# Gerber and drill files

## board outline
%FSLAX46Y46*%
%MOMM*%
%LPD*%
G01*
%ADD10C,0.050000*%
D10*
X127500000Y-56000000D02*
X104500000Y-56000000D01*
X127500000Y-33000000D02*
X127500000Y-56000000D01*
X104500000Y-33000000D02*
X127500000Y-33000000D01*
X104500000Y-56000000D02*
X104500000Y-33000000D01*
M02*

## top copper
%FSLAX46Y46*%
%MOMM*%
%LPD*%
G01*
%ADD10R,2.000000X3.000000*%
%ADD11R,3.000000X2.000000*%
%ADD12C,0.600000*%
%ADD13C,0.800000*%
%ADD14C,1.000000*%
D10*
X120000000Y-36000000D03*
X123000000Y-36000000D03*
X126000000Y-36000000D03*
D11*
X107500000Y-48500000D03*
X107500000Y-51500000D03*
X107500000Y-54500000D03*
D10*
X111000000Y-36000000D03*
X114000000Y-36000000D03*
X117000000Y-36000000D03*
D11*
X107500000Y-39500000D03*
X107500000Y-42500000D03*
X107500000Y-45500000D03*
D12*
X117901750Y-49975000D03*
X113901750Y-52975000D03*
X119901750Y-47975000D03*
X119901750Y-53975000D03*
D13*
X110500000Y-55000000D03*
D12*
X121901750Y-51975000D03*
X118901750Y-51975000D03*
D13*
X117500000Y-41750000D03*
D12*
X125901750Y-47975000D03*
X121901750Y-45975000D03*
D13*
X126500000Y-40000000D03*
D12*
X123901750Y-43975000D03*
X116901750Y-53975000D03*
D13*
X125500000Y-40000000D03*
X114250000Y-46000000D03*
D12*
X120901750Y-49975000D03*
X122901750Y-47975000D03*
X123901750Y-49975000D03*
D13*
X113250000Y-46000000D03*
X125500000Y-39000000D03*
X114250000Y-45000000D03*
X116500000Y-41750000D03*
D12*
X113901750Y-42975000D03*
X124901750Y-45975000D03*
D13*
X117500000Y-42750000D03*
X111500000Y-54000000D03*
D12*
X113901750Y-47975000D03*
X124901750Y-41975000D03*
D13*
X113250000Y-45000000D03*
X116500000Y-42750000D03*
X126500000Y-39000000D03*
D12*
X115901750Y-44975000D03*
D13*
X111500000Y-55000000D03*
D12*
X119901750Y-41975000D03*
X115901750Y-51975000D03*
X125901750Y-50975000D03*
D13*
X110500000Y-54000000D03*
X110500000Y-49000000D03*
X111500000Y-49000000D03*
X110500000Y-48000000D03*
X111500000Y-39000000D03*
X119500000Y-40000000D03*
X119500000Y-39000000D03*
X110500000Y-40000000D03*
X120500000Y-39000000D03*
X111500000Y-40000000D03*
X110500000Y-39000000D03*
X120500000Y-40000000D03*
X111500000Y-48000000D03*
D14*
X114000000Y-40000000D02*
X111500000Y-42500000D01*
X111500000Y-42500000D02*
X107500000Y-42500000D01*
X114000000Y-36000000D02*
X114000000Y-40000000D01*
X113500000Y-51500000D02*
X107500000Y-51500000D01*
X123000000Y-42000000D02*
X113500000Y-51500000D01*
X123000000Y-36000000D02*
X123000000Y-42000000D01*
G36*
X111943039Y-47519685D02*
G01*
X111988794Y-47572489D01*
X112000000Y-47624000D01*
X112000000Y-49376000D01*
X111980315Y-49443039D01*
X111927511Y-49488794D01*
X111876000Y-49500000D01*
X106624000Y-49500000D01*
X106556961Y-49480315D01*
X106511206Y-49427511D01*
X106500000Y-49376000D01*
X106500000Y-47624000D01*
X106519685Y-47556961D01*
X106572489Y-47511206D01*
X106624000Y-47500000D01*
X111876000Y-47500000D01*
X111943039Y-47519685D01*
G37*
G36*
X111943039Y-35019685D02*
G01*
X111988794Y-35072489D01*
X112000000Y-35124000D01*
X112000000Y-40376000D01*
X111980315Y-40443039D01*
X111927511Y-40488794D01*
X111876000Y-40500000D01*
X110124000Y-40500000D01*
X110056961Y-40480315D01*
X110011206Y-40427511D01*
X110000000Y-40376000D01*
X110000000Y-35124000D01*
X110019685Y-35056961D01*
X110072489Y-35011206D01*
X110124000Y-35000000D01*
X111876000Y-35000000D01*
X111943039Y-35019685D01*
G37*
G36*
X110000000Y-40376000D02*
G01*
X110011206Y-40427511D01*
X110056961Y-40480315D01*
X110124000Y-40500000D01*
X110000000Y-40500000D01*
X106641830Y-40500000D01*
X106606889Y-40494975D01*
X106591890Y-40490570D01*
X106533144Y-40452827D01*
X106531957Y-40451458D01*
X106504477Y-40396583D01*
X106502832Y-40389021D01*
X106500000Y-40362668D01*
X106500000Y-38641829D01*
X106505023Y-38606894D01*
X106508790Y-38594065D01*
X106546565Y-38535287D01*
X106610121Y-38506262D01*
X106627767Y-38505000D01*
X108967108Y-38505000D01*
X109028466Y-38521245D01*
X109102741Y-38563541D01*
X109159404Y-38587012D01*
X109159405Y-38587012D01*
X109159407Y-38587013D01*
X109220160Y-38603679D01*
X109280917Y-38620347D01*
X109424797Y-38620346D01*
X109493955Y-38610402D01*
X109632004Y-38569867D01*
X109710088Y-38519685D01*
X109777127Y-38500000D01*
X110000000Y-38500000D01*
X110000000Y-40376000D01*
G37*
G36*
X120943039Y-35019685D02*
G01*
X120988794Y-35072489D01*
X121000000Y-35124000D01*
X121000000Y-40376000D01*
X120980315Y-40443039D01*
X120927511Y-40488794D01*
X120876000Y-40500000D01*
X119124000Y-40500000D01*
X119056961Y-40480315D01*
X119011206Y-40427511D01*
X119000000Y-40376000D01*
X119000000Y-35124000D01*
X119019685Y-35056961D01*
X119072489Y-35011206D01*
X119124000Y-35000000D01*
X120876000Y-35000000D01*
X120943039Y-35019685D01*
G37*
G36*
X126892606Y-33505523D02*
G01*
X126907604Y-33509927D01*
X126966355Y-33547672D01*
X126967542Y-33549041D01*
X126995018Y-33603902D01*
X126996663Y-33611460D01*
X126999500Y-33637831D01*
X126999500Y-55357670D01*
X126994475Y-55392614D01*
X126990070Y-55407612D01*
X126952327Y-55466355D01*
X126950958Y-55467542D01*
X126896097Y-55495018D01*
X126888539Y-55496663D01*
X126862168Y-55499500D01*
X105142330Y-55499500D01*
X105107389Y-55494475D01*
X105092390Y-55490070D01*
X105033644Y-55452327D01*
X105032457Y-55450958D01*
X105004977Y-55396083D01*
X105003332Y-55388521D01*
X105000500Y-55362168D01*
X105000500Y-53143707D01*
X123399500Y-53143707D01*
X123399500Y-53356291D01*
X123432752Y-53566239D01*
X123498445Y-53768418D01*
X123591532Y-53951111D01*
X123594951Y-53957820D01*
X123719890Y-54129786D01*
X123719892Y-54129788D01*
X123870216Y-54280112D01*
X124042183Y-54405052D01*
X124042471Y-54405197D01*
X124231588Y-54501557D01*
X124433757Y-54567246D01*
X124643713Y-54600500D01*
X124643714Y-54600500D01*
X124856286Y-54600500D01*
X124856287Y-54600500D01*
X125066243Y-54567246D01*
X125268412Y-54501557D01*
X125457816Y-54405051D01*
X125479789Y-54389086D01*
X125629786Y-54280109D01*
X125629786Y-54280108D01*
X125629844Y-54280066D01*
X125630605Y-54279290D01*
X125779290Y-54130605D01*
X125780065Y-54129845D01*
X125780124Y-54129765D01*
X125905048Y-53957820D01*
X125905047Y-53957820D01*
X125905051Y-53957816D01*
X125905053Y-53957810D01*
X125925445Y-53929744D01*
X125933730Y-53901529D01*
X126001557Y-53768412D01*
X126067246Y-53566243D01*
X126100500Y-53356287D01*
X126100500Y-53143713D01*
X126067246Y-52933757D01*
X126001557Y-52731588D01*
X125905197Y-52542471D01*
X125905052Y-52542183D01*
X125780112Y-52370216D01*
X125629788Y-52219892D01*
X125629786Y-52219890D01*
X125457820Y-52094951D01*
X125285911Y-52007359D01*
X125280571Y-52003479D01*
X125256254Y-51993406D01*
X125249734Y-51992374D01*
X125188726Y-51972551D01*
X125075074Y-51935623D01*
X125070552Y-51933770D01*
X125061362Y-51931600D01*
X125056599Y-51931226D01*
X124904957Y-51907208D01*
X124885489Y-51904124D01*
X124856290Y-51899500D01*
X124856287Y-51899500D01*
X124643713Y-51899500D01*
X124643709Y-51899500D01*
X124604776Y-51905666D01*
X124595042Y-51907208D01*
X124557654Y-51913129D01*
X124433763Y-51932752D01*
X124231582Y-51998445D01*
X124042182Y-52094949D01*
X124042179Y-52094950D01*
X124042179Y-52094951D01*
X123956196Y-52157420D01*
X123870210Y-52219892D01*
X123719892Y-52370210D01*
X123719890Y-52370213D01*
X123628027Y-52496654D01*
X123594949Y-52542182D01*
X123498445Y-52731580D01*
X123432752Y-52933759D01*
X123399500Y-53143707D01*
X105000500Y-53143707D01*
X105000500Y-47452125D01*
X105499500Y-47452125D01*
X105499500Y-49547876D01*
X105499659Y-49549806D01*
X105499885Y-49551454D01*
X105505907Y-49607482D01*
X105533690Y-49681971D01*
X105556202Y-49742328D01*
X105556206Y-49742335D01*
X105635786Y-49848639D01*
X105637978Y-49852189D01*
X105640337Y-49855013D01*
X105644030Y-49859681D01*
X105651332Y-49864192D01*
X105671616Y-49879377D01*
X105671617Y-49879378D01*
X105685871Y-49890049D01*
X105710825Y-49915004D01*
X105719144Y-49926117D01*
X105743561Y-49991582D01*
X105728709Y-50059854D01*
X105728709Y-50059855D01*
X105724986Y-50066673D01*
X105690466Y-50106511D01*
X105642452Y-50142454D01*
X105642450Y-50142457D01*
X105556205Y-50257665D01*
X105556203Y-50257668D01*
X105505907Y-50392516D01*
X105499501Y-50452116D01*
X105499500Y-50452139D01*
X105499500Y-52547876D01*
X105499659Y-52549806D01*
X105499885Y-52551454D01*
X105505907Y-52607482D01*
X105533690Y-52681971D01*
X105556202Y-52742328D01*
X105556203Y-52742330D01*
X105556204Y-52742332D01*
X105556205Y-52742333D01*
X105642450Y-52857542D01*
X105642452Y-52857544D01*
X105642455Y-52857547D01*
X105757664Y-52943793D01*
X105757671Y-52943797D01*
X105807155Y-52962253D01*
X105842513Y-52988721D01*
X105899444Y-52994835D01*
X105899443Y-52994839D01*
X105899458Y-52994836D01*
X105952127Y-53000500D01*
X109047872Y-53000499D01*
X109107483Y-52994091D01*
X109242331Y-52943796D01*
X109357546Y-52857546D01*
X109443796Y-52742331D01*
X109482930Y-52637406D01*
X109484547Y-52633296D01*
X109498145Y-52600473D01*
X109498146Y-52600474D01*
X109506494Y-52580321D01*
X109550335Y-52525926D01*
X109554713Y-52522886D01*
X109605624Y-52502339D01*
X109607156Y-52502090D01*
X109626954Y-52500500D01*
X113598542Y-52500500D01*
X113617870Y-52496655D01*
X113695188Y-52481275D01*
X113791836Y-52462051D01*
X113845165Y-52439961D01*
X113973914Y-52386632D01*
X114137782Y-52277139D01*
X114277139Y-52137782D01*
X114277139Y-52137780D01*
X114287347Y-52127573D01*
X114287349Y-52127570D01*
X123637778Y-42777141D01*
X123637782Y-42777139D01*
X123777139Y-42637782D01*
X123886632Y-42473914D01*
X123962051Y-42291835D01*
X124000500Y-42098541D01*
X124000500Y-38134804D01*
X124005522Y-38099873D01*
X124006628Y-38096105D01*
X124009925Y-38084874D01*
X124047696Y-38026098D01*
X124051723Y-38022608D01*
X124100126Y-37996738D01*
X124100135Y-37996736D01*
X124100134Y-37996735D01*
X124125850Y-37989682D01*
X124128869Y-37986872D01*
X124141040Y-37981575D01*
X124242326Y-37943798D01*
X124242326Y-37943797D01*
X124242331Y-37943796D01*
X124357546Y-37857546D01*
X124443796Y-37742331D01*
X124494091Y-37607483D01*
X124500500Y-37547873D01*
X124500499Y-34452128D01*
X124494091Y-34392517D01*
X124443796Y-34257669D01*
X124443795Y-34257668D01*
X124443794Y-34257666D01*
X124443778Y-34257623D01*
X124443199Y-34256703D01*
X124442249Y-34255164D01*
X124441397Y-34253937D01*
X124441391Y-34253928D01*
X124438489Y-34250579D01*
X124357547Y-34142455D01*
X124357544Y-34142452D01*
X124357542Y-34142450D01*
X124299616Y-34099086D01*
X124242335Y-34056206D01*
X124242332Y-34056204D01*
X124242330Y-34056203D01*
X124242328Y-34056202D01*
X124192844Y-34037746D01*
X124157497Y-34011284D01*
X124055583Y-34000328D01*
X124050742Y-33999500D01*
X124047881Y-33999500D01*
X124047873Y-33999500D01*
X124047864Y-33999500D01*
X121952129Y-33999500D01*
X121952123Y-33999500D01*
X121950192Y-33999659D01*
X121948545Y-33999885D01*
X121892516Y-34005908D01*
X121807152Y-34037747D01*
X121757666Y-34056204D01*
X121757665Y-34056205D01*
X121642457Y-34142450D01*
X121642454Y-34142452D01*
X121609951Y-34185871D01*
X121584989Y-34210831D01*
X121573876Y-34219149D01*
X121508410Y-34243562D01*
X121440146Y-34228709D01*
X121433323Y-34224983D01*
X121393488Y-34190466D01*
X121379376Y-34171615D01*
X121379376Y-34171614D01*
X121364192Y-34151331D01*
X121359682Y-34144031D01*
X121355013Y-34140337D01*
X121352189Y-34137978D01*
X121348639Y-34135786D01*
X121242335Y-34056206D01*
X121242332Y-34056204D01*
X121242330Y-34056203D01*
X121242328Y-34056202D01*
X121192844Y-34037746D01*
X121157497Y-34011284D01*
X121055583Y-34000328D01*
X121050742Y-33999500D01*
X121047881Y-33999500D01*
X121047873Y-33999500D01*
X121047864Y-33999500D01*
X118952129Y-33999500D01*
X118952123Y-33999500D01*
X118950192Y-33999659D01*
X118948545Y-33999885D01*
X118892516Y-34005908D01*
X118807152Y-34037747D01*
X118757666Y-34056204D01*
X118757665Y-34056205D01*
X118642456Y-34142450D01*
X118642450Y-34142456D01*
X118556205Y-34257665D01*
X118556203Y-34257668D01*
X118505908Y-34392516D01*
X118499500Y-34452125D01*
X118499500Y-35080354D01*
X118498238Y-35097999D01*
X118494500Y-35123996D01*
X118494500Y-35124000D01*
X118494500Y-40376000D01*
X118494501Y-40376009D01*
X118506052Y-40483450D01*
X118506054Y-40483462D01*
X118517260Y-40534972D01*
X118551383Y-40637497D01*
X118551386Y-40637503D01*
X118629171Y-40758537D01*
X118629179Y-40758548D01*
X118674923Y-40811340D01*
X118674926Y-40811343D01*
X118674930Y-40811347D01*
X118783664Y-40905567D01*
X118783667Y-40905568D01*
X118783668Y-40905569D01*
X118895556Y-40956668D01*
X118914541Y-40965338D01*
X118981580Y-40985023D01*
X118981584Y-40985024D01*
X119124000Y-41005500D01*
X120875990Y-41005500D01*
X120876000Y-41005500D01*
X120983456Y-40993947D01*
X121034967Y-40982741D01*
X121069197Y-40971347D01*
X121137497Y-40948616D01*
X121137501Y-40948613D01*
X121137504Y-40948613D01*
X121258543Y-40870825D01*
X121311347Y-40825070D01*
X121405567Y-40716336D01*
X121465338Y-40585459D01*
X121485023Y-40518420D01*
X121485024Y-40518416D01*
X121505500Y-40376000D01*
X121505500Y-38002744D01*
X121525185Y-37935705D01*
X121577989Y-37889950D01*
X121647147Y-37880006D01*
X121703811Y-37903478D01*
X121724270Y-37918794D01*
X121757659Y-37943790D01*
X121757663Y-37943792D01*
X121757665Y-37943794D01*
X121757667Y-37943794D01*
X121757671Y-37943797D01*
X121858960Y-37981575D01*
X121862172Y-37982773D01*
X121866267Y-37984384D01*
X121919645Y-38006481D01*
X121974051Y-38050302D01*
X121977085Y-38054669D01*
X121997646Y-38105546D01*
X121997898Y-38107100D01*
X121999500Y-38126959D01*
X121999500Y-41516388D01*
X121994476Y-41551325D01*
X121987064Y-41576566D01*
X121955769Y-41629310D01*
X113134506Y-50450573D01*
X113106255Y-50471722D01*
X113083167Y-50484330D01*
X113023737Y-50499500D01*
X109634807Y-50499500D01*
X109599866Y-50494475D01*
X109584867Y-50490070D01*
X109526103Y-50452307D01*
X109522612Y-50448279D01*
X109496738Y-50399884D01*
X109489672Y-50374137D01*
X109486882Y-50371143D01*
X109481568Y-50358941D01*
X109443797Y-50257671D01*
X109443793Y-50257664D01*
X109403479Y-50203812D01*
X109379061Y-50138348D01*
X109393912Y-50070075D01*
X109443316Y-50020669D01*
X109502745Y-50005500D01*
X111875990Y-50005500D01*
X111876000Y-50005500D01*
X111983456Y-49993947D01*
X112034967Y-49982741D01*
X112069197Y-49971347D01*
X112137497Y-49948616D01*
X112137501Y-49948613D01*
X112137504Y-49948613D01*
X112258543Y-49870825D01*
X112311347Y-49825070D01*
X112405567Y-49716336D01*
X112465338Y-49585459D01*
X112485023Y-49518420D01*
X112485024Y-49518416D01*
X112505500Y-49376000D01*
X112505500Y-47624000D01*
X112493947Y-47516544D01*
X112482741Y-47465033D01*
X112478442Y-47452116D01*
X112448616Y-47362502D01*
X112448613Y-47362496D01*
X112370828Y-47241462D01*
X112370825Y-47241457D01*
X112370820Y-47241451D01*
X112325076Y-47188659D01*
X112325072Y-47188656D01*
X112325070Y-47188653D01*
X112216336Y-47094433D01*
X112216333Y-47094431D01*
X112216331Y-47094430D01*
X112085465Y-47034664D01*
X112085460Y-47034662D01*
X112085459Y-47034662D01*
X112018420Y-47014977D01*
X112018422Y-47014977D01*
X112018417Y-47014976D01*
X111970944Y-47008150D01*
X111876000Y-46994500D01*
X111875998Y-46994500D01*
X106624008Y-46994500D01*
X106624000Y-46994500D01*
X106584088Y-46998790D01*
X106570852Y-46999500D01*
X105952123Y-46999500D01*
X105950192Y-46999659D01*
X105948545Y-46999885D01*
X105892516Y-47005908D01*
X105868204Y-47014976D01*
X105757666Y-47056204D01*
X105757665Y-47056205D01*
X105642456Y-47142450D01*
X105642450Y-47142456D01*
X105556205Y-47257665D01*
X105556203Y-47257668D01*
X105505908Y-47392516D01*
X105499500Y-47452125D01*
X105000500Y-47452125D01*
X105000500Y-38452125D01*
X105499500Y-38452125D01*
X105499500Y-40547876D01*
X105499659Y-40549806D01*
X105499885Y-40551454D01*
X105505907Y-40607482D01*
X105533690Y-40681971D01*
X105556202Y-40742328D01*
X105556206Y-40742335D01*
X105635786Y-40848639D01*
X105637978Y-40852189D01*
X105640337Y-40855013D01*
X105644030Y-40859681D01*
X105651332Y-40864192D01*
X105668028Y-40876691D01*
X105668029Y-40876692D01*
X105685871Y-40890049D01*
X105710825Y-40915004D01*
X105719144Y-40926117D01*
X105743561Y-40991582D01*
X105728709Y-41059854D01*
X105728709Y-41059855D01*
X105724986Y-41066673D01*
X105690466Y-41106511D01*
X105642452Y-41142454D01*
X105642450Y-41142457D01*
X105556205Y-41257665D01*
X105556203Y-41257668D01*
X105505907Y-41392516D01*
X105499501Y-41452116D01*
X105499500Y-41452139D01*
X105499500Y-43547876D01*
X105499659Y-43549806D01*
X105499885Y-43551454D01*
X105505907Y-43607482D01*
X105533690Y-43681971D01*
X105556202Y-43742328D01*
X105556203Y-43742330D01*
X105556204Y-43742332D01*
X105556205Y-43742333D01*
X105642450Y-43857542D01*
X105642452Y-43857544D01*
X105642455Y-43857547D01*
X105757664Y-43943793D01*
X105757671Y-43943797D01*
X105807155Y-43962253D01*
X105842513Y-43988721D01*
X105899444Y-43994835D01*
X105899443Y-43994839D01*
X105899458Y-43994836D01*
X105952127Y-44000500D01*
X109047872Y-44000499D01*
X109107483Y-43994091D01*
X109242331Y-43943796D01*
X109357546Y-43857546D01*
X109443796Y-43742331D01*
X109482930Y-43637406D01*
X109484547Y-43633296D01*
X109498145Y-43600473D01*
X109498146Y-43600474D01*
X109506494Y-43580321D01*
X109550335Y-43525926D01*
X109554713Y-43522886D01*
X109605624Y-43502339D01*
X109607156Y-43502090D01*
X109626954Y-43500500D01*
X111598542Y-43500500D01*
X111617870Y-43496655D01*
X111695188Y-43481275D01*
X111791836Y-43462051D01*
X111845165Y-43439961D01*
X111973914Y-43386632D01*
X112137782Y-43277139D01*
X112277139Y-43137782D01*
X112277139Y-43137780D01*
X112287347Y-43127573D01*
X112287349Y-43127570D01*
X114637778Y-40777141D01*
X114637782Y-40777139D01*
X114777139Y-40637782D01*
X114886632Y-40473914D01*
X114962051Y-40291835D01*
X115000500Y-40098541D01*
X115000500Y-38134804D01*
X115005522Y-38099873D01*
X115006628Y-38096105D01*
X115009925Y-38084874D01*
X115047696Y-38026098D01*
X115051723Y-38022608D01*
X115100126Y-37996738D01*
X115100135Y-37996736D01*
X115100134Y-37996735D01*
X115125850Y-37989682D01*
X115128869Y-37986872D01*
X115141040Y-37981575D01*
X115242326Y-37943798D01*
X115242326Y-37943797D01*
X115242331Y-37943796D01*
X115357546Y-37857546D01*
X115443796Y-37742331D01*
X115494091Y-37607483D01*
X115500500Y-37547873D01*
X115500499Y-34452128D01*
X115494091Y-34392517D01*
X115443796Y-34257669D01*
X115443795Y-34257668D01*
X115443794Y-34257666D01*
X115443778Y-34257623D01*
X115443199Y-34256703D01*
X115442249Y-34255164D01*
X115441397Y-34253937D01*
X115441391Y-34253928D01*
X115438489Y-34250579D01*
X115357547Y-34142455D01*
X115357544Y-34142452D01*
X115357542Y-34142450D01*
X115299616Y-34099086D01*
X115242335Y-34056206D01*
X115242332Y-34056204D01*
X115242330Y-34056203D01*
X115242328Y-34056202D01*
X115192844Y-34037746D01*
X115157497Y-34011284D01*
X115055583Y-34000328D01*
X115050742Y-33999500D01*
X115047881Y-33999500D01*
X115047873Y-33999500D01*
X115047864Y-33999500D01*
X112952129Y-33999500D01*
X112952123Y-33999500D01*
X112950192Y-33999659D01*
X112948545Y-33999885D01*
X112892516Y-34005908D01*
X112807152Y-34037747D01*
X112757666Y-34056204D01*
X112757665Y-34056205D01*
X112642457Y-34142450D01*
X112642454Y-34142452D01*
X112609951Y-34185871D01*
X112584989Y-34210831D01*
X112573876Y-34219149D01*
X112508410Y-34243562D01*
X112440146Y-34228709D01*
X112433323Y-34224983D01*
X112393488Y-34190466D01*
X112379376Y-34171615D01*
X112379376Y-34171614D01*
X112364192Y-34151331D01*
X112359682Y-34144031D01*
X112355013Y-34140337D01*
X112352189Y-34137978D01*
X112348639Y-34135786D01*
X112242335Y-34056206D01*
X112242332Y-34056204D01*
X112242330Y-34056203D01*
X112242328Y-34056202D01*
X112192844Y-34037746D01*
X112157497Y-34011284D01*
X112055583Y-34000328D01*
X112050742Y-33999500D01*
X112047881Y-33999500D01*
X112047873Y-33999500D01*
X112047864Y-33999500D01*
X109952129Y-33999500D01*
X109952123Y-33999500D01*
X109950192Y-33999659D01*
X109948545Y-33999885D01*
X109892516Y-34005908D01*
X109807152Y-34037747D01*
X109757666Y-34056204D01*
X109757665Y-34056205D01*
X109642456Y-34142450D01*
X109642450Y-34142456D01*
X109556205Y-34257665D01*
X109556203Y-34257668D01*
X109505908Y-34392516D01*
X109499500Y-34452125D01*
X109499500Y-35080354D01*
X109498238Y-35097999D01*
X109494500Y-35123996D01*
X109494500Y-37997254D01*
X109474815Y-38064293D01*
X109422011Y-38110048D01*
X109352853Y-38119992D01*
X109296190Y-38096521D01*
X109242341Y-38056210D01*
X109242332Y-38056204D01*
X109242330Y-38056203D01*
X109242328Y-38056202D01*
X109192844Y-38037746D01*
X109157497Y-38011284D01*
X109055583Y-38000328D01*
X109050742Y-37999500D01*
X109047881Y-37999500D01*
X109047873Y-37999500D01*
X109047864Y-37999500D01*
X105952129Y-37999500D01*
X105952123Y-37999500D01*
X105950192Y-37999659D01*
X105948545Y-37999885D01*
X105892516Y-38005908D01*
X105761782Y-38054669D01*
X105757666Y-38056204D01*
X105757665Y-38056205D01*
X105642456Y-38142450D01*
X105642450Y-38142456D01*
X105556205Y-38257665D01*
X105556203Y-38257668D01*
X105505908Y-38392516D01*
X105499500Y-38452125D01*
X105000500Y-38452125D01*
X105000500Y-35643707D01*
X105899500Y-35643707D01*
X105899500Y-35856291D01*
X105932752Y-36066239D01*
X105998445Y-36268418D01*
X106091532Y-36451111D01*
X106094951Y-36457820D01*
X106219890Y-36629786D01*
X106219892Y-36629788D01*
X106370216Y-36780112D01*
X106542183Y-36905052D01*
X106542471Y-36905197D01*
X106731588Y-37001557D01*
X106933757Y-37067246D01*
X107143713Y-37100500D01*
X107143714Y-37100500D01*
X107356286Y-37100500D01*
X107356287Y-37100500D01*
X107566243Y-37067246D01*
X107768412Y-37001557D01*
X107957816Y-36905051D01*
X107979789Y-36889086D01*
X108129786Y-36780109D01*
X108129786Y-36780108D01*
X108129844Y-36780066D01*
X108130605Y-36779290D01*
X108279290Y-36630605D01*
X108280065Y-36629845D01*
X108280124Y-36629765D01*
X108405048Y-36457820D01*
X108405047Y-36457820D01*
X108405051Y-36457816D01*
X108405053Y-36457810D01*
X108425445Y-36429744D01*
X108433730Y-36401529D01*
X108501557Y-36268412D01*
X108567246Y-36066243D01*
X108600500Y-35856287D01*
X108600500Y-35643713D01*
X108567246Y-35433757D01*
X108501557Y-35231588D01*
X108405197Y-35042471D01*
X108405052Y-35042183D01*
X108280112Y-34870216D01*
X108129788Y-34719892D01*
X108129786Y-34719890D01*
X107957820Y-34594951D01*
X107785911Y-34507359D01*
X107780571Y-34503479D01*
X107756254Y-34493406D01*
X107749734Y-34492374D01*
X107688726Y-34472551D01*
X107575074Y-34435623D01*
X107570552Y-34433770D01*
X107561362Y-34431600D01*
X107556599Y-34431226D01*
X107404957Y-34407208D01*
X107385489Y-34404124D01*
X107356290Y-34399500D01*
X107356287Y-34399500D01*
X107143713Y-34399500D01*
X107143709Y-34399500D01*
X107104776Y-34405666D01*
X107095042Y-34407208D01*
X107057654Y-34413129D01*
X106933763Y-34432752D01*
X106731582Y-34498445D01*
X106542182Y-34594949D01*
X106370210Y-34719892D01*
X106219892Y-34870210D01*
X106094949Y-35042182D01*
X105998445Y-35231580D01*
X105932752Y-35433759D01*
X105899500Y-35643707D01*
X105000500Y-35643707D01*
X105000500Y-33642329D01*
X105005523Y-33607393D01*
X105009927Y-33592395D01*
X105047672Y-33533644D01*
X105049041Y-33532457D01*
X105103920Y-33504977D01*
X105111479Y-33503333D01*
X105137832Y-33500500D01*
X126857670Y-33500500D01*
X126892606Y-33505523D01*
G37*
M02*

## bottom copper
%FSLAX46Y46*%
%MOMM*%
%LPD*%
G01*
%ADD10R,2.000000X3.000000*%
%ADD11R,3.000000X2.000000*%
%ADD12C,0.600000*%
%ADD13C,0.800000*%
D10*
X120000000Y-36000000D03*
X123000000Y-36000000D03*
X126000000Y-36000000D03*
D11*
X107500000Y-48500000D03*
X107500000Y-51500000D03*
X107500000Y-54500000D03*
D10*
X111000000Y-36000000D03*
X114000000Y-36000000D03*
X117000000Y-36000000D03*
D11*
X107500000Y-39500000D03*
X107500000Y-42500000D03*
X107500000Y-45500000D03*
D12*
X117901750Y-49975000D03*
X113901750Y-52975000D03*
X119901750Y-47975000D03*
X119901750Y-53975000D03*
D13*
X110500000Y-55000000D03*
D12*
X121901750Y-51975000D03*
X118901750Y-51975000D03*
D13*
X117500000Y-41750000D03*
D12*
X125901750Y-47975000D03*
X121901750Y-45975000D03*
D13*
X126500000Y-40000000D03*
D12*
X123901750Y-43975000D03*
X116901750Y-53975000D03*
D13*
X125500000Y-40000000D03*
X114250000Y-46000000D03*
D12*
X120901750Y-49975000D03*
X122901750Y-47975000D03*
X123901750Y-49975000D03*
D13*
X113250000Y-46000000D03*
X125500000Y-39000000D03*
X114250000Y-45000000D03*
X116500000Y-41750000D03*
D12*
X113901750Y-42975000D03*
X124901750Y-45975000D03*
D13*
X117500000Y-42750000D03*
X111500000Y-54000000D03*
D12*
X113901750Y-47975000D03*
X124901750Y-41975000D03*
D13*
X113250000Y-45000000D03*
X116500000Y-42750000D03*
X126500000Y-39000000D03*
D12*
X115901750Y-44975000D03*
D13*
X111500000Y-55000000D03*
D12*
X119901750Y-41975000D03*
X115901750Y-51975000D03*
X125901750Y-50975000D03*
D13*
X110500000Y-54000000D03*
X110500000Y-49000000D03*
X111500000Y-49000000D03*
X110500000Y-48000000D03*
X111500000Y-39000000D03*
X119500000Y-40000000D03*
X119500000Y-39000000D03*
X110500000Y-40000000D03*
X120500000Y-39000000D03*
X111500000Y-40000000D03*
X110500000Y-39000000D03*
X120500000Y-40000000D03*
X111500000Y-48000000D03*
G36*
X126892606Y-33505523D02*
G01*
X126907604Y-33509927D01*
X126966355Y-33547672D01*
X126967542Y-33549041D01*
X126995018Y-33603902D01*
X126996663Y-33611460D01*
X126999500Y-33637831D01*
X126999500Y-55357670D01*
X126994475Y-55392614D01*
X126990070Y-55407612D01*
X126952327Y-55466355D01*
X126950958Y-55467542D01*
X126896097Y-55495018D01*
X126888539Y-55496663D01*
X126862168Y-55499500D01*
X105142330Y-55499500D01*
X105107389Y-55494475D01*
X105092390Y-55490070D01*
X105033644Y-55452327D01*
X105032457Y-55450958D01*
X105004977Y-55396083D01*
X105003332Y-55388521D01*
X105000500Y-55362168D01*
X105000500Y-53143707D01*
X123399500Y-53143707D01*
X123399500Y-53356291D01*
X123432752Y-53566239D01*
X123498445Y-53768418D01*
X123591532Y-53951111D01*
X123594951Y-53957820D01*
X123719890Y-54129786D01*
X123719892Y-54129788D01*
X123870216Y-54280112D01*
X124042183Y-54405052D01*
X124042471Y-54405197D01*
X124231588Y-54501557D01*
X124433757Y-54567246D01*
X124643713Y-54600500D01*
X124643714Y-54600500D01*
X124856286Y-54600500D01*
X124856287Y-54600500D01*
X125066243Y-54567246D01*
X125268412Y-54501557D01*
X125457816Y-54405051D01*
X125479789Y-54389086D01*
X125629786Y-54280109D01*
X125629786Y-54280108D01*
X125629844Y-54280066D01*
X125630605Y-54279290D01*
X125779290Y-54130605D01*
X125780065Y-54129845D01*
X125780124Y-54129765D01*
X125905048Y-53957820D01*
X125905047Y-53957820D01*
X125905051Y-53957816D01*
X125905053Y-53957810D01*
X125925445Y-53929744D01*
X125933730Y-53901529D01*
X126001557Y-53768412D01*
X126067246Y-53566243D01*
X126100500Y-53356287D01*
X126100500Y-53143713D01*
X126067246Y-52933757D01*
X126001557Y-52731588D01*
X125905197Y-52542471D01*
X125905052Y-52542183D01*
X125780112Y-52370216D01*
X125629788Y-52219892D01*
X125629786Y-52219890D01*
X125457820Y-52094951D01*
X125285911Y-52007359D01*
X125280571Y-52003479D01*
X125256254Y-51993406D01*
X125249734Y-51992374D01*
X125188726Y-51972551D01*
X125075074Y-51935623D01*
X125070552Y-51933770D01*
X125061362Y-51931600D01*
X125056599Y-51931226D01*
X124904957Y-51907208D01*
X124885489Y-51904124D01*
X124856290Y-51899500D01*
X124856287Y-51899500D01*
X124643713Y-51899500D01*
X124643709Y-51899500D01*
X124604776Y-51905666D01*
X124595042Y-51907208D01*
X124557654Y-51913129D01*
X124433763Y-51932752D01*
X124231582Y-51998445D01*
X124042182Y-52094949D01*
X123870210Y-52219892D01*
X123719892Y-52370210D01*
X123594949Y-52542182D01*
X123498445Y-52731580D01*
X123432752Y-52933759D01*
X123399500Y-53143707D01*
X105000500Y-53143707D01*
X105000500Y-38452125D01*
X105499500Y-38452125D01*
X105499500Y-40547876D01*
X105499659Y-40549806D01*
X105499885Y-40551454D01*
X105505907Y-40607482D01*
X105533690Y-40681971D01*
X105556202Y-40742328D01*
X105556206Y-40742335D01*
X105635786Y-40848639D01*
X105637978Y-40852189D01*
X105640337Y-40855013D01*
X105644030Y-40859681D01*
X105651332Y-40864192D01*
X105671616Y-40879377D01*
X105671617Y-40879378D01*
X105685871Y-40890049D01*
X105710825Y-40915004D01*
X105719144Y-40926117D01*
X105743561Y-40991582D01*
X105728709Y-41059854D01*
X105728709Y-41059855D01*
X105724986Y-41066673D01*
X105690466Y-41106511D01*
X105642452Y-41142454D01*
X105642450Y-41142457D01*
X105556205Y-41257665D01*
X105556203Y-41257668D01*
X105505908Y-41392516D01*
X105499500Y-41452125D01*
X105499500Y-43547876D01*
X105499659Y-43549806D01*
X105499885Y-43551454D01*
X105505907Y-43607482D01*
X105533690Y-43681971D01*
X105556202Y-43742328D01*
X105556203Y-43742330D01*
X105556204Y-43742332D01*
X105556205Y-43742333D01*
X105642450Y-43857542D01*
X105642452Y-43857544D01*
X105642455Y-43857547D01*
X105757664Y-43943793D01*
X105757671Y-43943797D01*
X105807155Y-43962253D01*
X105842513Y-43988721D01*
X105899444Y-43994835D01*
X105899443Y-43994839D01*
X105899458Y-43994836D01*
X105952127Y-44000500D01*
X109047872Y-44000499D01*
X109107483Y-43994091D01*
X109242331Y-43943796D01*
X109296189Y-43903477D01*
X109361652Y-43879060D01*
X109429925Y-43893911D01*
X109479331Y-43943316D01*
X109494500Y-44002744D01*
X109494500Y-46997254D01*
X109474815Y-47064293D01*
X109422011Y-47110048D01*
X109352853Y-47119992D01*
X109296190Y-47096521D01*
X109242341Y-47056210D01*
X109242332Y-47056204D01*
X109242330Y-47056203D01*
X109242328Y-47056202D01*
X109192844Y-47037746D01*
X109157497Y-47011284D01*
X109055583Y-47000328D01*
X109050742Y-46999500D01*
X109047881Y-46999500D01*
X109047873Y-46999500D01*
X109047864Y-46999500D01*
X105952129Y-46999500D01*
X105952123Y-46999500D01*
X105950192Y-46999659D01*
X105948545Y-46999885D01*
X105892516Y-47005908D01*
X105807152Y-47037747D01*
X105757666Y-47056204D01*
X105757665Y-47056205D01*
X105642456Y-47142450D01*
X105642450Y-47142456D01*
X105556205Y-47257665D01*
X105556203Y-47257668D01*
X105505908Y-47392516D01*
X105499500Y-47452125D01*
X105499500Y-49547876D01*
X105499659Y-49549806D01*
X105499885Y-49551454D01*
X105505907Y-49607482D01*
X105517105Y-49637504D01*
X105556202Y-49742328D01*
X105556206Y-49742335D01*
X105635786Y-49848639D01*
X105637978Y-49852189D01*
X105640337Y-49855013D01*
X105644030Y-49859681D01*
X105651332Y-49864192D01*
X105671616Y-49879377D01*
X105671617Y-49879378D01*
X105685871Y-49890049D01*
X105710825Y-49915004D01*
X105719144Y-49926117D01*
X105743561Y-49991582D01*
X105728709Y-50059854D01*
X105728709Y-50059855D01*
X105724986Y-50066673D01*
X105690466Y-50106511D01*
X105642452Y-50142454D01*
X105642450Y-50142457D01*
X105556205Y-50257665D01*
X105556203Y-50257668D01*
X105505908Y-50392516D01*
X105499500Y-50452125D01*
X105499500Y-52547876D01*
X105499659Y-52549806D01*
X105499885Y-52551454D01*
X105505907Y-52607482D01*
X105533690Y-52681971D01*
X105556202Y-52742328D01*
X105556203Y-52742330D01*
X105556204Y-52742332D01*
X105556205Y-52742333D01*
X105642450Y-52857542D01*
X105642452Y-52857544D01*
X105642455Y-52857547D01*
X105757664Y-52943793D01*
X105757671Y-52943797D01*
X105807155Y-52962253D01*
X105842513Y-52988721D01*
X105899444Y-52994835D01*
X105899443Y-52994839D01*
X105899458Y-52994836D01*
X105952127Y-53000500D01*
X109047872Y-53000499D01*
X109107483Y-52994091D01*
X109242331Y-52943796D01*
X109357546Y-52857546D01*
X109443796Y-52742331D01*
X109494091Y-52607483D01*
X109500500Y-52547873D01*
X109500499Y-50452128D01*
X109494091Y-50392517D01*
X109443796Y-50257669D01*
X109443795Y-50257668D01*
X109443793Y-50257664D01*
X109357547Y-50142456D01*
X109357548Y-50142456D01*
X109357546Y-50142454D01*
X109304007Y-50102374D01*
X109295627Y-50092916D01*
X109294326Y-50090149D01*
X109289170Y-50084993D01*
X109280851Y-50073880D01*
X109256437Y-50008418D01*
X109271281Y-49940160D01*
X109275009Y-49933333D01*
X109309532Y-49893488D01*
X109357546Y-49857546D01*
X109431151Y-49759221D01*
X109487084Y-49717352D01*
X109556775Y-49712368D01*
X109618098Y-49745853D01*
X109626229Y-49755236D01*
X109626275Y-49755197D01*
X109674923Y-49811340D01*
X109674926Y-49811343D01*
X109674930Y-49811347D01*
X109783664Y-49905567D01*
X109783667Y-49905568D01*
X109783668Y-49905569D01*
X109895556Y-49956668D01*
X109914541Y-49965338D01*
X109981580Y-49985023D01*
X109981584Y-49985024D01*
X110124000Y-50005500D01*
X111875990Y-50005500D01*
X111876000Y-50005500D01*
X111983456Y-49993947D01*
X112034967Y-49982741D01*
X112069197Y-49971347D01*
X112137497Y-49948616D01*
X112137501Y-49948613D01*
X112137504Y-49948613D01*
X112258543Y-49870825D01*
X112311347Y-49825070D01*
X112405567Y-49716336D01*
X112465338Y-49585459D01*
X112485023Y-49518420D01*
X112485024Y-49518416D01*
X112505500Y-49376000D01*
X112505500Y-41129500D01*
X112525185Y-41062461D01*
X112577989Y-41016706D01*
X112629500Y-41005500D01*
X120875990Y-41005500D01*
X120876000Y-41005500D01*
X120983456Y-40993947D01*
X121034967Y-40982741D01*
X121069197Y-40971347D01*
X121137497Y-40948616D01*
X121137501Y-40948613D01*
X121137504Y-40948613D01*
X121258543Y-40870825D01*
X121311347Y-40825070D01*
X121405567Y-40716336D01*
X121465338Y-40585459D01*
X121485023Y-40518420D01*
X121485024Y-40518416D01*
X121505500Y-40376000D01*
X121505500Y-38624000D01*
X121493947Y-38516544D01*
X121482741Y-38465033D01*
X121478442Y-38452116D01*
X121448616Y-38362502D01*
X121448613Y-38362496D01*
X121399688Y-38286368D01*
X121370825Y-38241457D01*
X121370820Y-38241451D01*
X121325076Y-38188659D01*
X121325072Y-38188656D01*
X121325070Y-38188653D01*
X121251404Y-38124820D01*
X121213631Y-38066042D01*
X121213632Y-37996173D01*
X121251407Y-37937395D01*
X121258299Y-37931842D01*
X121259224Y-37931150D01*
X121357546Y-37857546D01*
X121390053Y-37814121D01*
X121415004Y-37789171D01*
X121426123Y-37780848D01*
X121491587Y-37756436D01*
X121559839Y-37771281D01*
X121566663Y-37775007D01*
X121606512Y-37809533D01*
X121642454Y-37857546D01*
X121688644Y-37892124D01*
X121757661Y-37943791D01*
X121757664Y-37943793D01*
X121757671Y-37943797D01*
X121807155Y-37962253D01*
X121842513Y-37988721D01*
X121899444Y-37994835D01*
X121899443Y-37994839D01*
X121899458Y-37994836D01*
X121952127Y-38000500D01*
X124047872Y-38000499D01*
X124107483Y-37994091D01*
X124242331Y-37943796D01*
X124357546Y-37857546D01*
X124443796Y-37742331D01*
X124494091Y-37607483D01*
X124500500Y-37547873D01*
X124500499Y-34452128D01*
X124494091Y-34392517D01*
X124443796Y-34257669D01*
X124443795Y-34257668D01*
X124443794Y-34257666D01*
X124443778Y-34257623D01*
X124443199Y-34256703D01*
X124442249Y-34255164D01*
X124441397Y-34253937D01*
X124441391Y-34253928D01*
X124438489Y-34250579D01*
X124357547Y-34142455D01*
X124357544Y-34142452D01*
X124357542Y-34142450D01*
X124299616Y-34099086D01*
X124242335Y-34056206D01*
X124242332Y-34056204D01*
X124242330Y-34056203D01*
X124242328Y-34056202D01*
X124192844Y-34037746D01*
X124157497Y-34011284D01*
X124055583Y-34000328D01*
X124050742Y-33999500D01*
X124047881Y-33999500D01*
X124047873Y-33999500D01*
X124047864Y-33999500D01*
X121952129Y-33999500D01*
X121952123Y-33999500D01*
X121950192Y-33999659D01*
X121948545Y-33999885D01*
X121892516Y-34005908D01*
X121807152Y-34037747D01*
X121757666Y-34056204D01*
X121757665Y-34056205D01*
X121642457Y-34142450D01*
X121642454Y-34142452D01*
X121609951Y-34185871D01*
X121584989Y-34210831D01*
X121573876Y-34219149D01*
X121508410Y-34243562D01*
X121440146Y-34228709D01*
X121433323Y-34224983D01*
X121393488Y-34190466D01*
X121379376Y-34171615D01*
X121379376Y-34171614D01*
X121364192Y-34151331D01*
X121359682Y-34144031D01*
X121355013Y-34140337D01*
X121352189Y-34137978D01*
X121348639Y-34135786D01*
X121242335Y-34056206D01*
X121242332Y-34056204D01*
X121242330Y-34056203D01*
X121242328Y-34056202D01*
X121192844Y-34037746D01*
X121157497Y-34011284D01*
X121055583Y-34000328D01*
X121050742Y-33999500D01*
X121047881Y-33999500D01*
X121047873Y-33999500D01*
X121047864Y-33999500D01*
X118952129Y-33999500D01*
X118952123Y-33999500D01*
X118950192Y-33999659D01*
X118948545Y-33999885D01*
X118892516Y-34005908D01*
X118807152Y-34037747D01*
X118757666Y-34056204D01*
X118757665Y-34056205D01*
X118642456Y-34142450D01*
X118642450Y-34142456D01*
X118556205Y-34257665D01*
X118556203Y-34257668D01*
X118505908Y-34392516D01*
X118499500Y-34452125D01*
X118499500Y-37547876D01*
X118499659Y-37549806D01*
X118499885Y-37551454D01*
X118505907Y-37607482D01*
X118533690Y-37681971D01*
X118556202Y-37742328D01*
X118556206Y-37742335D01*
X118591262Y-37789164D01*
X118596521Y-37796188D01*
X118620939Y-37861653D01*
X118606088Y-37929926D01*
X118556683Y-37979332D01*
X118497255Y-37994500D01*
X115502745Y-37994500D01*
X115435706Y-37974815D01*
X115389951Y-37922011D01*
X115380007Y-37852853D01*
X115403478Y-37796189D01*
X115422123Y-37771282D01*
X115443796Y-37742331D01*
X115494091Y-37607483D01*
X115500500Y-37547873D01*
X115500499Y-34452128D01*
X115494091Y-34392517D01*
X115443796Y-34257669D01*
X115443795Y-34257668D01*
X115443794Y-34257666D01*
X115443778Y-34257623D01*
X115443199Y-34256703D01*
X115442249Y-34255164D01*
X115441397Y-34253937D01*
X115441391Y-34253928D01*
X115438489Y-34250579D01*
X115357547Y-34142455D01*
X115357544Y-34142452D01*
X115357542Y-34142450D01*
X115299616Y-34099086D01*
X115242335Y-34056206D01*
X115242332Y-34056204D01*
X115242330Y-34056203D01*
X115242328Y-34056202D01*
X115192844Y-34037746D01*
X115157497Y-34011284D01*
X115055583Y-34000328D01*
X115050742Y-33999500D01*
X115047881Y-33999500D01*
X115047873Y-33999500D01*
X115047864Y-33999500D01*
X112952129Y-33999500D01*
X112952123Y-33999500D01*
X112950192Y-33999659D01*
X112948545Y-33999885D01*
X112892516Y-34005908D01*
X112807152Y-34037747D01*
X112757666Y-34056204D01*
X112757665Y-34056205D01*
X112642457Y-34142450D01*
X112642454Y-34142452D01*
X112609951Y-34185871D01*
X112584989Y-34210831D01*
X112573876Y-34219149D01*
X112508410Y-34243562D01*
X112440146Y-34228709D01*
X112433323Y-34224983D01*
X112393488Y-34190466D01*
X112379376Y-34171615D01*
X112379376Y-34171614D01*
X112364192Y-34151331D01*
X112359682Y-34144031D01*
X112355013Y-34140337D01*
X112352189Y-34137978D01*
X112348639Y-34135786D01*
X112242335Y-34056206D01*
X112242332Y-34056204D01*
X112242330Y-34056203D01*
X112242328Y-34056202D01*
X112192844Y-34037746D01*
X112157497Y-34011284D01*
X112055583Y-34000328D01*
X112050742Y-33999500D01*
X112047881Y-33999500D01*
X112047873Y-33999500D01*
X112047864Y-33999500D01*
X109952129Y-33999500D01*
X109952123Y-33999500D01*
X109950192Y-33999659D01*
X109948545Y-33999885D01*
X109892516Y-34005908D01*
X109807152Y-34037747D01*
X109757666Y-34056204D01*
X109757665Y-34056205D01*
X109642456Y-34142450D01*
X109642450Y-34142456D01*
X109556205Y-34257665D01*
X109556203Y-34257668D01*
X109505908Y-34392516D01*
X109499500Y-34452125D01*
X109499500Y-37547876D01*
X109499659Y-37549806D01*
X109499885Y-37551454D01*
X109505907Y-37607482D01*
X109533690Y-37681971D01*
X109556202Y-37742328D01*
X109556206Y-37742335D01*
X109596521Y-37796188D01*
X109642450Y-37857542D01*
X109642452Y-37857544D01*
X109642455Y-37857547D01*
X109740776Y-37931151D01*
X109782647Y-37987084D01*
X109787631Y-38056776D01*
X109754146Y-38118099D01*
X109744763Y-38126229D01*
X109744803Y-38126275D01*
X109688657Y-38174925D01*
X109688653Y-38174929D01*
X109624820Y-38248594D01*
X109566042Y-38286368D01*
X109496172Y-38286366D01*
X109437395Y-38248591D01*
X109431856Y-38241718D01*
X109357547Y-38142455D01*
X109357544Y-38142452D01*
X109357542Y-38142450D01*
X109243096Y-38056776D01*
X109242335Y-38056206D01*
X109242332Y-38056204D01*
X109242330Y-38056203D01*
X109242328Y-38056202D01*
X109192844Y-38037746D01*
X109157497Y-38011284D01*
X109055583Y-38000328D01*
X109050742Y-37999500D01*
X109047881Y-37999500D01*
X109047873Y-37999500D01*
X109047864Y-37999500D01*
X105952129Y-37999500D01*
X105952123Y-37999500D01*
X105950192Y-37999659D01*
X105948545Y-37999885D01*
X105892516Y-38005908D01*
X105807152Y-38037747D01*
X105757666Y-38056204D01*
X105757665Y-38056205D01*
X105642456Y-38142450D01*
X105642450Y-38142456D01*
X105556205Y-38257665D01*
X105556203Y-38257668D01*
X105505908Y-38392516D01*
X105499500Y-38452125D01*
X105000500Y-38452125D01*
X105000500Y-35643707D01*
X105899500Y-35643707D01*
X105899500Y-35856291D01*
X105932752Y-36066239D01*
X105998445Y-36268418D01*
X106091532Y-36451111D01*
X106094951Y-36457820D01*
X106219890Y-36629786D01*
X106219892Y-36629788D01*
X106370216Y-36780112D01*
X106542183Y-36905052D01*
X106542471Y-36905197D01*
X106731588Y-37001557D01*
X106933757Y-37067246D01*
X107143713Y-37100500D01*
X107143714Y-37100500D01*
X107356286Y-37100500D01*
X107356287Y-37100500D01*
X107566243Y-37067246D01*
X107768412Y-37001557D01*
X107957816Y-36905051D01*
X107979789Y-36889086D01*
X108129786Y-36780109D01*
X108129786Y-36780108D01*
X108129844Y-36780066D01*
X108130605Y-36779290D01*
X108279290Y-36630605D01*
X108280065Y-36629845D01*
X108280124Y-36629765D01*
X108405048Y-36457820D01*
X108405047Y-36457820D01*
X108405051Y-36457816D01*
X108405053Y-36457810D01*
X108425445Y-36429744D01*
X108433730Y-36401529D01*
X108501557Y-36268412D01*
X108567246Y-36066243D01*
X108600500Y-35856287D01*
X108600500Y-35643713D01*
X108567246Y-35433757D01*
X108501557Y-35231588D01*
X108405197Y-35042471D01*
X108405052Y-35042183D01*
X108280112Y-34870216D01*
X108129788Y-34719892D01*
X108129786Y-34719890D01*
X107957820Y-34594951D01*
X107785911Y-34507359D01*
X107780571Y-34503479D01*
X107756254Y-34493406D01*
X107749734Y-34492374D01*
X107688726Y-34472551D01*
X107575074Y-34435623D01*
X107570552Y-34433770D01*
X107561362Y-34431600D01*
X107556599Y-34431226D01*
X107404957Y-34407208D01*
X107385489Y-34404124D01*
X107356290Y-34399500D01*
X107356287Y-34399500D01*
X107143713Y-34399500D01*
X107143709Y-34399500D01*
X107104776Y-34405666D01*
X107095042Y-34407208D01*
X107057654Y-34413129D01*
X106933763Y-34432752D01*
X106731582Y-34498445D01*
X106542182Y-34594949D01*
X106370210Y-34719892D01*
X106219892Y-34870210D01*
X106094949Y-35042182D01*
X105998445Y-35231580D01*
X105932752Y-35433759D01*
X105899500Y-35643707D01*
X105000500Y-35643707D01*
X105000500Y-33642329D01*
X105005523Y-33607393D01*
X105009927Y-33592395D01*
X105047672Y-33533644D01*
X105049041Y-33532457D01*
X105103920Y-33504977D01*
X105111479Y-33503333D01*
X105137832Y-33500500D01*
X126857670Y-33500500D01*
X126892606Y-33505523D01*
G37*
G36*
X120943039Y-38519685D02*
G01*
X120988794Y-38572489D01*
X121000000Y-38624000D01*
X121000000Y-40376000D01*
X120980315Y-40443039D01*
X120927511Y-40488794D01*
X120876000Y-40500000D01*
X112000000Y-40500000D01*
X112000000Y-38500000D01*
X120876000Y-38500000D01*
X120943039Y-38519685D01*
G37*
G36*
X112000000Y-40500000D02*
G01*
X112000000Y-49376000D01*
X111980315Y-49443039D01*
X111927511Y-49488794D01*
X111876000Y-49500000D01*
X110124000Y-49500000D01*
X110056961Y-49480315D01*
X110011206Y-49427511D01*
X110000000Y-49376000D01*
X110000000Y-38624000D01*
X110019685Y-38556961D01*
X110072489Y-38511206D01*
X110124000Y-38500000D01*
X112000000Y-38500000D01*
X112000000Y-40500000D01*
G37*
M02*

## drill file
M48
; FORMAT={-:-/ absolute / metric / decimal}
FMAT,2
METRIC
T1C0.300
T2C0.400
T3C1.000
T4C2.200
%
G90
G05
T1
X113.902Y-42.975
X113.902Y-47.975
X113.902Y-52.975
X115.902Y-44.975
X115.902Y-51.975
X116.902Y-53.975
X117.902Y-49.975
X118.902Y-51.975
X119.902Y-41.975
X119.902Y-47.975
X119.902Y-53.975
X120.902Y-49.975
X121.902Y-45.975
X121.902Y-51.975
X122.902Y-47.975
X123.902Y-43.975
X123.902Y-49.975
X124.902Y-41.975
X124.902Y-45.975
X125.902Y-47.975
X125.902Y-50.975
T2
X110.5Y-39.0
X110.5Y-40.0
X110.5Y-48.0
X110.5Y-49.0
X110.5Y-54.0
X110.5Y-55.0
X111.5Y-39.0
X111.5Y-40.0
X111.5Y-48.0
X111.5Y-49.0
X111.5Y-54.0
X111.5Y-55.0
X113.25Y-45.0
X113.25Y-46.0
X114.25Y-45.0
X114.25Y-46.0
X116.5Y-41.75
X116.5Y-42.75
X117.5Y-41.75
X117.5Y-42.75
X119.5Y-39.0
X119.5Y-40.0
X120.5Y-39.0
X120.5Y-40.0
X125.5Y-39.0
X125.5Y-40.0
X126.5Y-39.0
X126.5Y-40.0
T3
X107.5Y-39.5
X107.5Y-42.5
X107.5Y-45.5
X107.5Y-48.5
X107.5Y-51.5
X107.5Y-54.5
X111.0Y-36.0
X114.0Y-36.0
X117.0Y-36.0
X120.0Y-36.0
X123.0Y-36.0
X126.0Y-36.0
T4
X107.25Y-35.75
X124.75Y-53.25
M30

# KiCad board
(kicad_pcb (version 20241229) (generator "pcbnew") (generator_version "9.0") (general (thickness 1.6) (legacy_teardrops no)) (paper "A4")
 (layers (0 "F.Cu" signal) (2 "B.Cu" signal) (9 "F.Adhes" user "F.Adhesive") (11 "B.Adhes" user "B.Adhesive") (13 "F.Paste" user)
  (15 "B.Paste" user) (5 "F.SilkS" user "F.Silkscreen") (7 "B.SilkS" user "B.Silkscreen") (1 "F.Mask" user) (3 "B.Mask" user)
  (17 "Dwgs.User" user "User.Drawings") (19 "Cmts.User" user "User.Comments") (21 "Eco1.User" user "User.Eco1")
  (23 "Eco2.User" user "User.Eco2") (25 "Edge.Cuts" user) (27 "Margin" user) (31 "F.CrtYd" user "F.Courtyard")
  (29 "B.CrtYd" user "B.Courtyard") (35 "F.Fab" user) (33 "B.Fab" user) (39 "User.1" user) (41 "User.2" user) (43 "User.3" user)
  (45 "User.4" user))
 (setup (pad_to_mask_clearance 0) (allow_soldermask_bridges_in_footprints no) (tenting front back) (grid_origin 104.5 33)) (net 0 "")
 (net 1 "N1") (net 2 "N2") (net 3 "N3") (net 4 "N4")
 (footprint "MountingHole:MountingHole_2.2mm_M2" (layer "F.Cu") (at 107.25 35.75)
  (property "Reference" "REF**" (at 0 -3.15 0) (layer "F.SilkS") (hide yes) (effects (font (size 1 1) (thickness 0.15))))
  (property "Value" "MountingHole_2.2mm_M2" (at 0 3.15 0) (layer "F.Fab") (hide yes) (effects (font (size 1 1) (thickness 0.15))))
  (pad "" np_thru_hole circle (at 0 0) (size 2.2 2.2) (drill 2.2) (layers "*.Cu" "*.Mask")))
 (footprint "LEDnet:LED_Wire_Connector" (layer "F.Cu") (at 123 36)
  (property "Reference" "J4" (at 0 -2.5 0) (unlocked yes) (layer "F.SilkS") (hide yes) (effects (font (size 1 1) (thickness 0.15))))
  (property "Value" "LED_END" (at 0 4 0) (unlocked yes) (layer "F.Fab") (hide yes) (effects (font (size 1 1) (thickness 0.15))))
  (pad "1" thru_hole rect (at -3 0) (size 2 3) (drill 1) (layers "*.Cu" "*.Mask") (remove_unused_layers no) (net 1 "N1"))
  (pad "2" thru_hole rect (at 0 0) (size 2 3) (drill 1) (layers "*.Cu" "*.Mask") (remove_unused_layers no) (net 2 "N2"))
  (pad "3" thru_hole rect (at 3 0) (size 2 3) (drill 1) (layers "*.Cu" "*.Mask") (remove_unused_layers no) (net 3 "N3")))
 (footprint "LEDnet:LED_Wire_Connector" (layer "F.Cu") (at 107.5 51.5 -90)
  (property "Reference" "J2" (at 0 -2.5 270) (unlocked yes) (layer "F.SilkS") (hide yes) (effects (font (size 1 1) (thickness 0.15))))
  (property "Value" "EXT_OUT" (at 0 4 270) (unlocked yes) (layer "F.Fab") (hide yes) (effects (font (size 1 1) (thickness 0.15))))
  (pad "1" thru_hole rect (at -3 0 270) (size 2 3) (drill 1) (layers "*.Cu" "*.Mask") (remove_unused_layers no) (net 1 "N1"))
  (pad "2" thru_hole rect (at 0 0 270) (size 2 3) (drill 1) (layers "*.Cu" "*.Mask") (remove_unused_layers no) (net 2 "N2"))
  (pad "3" thru_hole rect (at 3 0 270) (size 2 3) (drill 1) (layers "*.Cu" "*.Mask") (remove_unused_layers no) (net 3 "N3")))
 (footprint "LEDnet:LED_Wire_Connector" (layer "F.Cu") (at 114 36)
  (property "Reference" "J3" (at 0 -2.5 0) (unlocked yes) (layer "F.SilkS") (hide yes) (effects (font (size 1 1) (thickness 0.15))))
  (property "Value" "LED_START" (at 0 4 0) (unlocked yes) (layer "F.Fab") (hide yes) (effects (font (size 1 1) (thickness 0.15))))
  (pad "1" thru_hole rect (at -3 0) (size 2 3) (drill 1) (layers "*.Cu" "*.Mask") (remove_unused_layers no) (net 1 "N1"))
  (pad "2" thru_hole rect (at 0 0) (size 2 3) (drill 1) (layers "*.Cu" "*.Mask") (remove_unused_layers no) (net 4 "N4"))
  (pad "3" thru_hole rect (at 3 0) (size 2 3) (drill 1) (layers "*.Cu" "*.Mask") (remove_unused_layers no) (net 3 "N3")))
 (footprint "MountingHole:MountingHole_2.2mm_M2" (layer "F.Cu") (at 124.75 53.25)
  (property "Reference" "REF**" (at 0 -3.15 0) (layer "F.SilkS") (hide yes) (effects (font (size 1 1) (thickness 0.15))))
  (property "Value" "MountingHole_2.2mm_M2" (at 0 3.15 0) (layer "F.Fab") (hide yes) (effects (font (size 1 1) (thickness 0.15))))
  (pad "" np_thru_hole circle (at 0 0) (size 2.2 2.2) (drill 2.2) (layers "*.Cu" "*.Mask")))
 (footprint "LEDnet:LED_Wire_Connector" (layer "F.Cu") (at 107.5 42.5 -90)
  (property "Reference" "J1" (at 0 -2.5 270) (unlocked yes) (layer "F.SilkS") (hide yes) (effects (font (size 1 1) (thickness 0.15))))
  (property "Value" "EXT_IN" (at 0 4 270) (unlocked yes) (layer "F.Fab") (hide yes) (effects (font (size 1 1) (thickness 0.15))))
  (pad "1" thru_hole rect (at -3 0 270) (size 2 3) (drill 1) (layers "*.Cu" "*.Mask") (remove_unused_layers no) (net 1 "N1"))
  (pad "2" thru_hole rect (at 0 0 270) (size 2 3) (drill 1) (layers "*.Cu" "*.Mask") (remove_unused_layers no) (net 4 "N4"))
  (pad "3" thru_hole rect (at 3 0 270) (size 2 3) (drill 1) (layers "*.Cu" "*.Mask") (remove_unused_layers no) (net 3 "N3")))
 (gr_line (start 127.5 56) (end 104.5 56) (stroke (width 0.05) (type default)) (layer "Edge.Cuts"))
 (gr_line (start 127.5 33) (end 127.5 56) (stroke (width 0.05) (type default)) (layer "Edge.Cuts"))
 (gr_line (start 104.5 33) (end 127.5 33) (stroke (width 0.05) (type default)) (layer "Edge.Cuts"))
 (gr_line (start 104.5 56) (end 104.5 33) (stroke (width 0.05) (type default)) (layer "Edge.Cuts"))
 (segment (start 114 40) (end 111.5 42.5) (width 1) (layer "F.Cu") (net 4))
 (segment (start 111.5 42.5) (end 107.5 42.5) (width 1) (layer "F.Cu") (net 4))
 (segment (start 114 36) (end 114 40) (width 1) (layer "F.Cu") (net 4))
 (via (at 117.90175 49.975) (size 0.6) (drill 0.3) (layers "F.Cu" "B.Cu") (free yes) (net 3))
 (via (at 113.90175 52.975) (size 0.6) (drill 0.3) (layers "F.Cu" "B.Cu") (free yes) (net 3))
 (via (at 119.90175 47.975) (size 0.6) (drill 0.3) (layers "F.Cu" "B.Cu") (free yes) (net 3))
 (via (at 119.90175 53.975) (size 0.6) (drill 0.3) (layers "F.Cu" "B.Cu") (free yes) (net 3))
 (via (at 110.5 55) (size 0.8) (drill 0.4) (layers "F.Cu" "B.Cu") (free yes) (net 3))
 (via (at 121.90175 51.975) (size 0.6) (drill 0.3) (layers "F.Cu" "B.Cu") (free yes) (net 3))
 (via (at 118.90175 51.975) (size 0.6) (drill 0.3) (layers "F.Cu" "B.Cu") (free yes) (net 3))
 (via (at 117.5 41.75) (size 0.8) (drill 0.4) (layers "F.Cu" "B.Cu") (free yes) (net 3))
 (via (at 125.90175 47.975) (size 0.6) (drill 0.3) (layers "F.Cu" "B.Cu") (free yes) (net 3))
 (via (at 121.90175 45.975) (size 0.6) (drill 0.3) (layers "F.Cu" "B.Cu") (free yes) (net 3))
 (via (at 126.5 40) (size 0.8) (drill 0.4) (layers "F.Cu" "B.Cu") (free yes) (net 3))
 (via (at 123.90175 43.975) (size 0.6) (drill 0.3) (layers "F.Cu" "B.Cu") (free yes) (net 3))
 (via (at 116.90175 53.975) (size 0.6) (drill 0.3) (layers "F.Cu" "B.Cu") (free yes) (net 3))
 (via (at 125.5 40) (size 0.8) (drill 0.4) (layers "F.Cu" "B.Cu") (free yes) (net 3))
 (via (at 114.25 46) (size 0.8) (drill 0.4) (layers "F.Cu" "B.Cu") (free yes) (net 3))
 (via (at 120.90175 49.975) (size 0.6) (drill 0.3) (layers "F.Cu" "B.Cu") (free yes) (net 3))
 (via (at 122.90175 47.975) (size 0.6) (drill 0.3) (layers "F.Cu" "B.Cu") (free yes) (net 3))
 (via (at 123.90175 49.975) (size 0.6) (drill 0.3) (layers "F.Cu" "B.Cu") (free yes) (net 3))
 (via (at 113.25 46) (size 0.8) (drill 0.4) (layers "F.Cu" "B.Cu") (free yes) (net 3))
 (via (at 125.5 39) (size 0.8) (drill 0.4) (layers "F.Cu" "B.Cu") (free yes) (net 3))
 (via (at 114.25 45) (size 0.8) (drill 0.4) (layers "F.Cu" "B.Cu") (free yes) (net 3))
 (via (at 116.5 41.75) (size 0.8) (drill 0.4) (layers "F.Cu" "B.Cu") (free yes) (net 3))
 (via (at 113.90175 42.975) (size 0.6) (drill 0.3) (layers "F.Cu" "B.Cu") (free yes) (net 3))
 (via (at 124.90175 45.975) (size 0.6) (drill 0.3) (layers "F.Cu" "B.Cu") (free yes) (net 3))
 (via (at 117.5 42.75) (size 0.8) (drill 0.4) (layers "F.Cu" "B.Cu") (free yes) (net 3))
 (via (at 111.5 54) (size 0.8) (drill 0.4) (layers "F.Cu" "B.Cu") (free yes) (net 3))
 (via (at 113.90175 47.975) (size 0.6) (drill 0.3) (layers "F.Cu" "B.Cu") (free yes) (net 3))
 (via (at 124.90175 41.975) (size 0.6) (drill 0.3) (layers "F.Cu" "B.Cu") (free yes) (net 3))
 (via (at 113.25 45) (size 0.8) (drill 0.4) (layers "F.Cu" "B.Cu") (free yes) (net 3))
 (via (at 116.5 42.75) (size 0.8) (drill 0.4) (layers "F.Cu" "B.Cu") (free yes) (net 3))
 (via (at 126.5 39) (size 0.8) (drill 0.4) (layers "F.Cu" "B.Cu") (free yes) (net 3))
 (via (at 115.90175 44.975) (size 0.6) (drill 0.3) (layers "F.Cu" "B.Cu") (free yes) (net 3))
 (via (at 111.5 55) (size 0.8) (drill 0.4) (layers "F.Cu" "B.Cu") (free yes) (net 3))
 (via (at 119.90175 41.975) (size 0.6) (drill 0.3) (layers "F.Cu" "B.Cu") (free yes) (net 3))
 (via (at 115.90175 51.975) (size 0.6) (drill 0.3) (layers "F.Cu" "B.Cu") (free yes) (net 3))
 (via (at 125.90175 50.975) (size 0.6) (drill 0.3) (layers "F.Cu" "B.Cu") (free yes) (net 3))
 (via (at 110.5 54) (size 0.8) (drill 0.4) (layers "F.Cu" "B.Cu") (free yes) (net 3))
 (via (at 110.5 49) (size 0.8) (drill 0.4) (layers "F.Cu" "B.Cu") (free yes)
  (teardrops (best_length_ratio 0.5) (max_length 1) (best_width_ratio 1) (max_width 2) (curved_edges no) (filter_ratio 0.9) (enabled yes)
   (allow_two_segments yes) (prefer_zone_connections yes))
  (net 1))
 (via (at 111.5 49) (size 0.8) (drill 0.4) (layers "F.Cu" "B.Cu") (free yes)
  (teardrops (best_length_ratio 0.5) (max_length 1) (best_width_ratio 1) (max_width 2) (curved_edges no) (filter_ratio 0.9) (enabled yes)
   (allow_two_segments yes) (prefer_zone_connections yes))
  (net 1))
 (via (at 110.5 48) (size 0.8) (drill 0.4) (layers "F.Cu" "B.Cu") (free yes)
  (teardrops (best_length_ratio 0.5) (max_length 1) (best_width_ratio 1) (max_width 2) (curved_edges no) (filter_ratio 0.9) (enabled yes)
   (allow_two_segments yes) (prefer_zone_connections yes))
  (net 1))
 (via (at 111.5 39) (size 0.8) (drill 0.4) (layers "F.Cu" "B.Cu") (free yes)
  (teardrops (best_length_ratio 0.5) (max_length 1) (best_width_ratio 1) (max_width 2) (curved_edges no) (filter_ratio 0.9) (enabled yes)
   (allow_two_segments yes) (prefer_zone_connections yes))
  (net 1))
 (via (at 119.5 40) (size 0.8) (drill 0.4) (layers "F.Cu" "B.Cu") (free yes)
  (teardrops (best_length_ratio 0.5) (max_length 1) (best_width_ratio 1) (max_width 2) (curved_edges no) (filter_ratio 0.9) (enabled yes)
   (allow_two_segments yes) (prefer_zone_connections yes))
  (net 1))
 (via (at 119.5 39) (size 0.8) (drill 0.4) (layers "F.Cu" "B.Cu") (free yes)
  (teardrops (best_length_ratio 0.5) (max_length 1) (best_width_ratio 1) (max_width 2) (curved_edges no) (filter_ratio 0.9) (enabled yes)
   (allow_two_segments yes) (prefer_zone_connections yes))
  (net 1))
 (via (at 110.5 40) (size 0.8) (drill 0.4) (layers "F.Cu" "B.Cu") (free yes)
  (teardrops (best_length_ratio 0.5) (max_length 1) (best_width_ratio 1) (max_width 2) (curved_edges no) (filter_ratio 0.9) (enabled yes)
   (allow_two_segments yes) (prefer_zone_connections yes))
  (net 1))
 (via (at 120.5 39) (size 0.8) (drill 0.4) (layers "F.Cu" "B.Cu") (free yes)
  (teardrops (best_length_ratio 0.5) (max_length 1) (best_width_ratio 1) (max_width 2) (curved_edges no) (filter_ratio 0.9) (enabled yes)
   (allow_two_segments yes) (prefer_zone_connections yes))
  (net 1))
 (via (at 111.5 40) (size 0.8) (drill 0.4) (layers "F.Cu" "B.Cu") (free yes)
  (teardrops (best_length_ratio 0.5) (max_length 1) (best_width_ratio 1) (max_width 2) (curved_edges no) (filter_ratio 0.9) (enabled yes)
   (allow_two_segments yes) (prefer_zone_connections yes))
  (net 1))
 (via (at 110.5 39) (size 0.8) (drill 0.4) (layers "F.Cu" "B.Cu") (free yes)
  (teardrops (best_length_ratio 0.5) (max_length 1) (best_width_ratio 1) (max_width 2) (curved_edges no) (filter_ratio 0.9) (enabled yes)
   (allow_two_segments yes) (prefer_zone_connections yes))
  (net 1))
 (via (at 120.5 40) (size 0.8) (drill 0.4) (layers "F.Cu" "B.Cu") (free yes)
  (teardrops (best_length_ratio 0.5) (max_length 1) (best_width_ratio 1) (max_width 2) (curved_edges no) (filter_ratio 0.9) (enabled yes)
   (allow_two_segments yes) (prefer_zone_connections yes))
  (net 1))
 (via (at 111.5 48) (size 0.8) (drill 0.4) (layers "F.Cu" "B.Cu") (free yes)
  (teardrops (best_length_ratio 0.5) (max_length 1) (best_width_ratio 1) (max_width 2) (curved_edges no) (filter_ratio 0.9) (enabled yes)
   (allow_two_segments yes) (prefer_zone_connections yes))
  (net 1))
 (segment (start 113.5 51.5) (end 107.5 51.5) (width 1) (layer "F.Cu") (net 2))
 (segment (start 123 42) (end 113.5 51.5) (width 1) (layer "F.Cu") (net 2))
 (segment (start 123 36) (end 123 42) (width 1) (layer "F.Cu") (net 2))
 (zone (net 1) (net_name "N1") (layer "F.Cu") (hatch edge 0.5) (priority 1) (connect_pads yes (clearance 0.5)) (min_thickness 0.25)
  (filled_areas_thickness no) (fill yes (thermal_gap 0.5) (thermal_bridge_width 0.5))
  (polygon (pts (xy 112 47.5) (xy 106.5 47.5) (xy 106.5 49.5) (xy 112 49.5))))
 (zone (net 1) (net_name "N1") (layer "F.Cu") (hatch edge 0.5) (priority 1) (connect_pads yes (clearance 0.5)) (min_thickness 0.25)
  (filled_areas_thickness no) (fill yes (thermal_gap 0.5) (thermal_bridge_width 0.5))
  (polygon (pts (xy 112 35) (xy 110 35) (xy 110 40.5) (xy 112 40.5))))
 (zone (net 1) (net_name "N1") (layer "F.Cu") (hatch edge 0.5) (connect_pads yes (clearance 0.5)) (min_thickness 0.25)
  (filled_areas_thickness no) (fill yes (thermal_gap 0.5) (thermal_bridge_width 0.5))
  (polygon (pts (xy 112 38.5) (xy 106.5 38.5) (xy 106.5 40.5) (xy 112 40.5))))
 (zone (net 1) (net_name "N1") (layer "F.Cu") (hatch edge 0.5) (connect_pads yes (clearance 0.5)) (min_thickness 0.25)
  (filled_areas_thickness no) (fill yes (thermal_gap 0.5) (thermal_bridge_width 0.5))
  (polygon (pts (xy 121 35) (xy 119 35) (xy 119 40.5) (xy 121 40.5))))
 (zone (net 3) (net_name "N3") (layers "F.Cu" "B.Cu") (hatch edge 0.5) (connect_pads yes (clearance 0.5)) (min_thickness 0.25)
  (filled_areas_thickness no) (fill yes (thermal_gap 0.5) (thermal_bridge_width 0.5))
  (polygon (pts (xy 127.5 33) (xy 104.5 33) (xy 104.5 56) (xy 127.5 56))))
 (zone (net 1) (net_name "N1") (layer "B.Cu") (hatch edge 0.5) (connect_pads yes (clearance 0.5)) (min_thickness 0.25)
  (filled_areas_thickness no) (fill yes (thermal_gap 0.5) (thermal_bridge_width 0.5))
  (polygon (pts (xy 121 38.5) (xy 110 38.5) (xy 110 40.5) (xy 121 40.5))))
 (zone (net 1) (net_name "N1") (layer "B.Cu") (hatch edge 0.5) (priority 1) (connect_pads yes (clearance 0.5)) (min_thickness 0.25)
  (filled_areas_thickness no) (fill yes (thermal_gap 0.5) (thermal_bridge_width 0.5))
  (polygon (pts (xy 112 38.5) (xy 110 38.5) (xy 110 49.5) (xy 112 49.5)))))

